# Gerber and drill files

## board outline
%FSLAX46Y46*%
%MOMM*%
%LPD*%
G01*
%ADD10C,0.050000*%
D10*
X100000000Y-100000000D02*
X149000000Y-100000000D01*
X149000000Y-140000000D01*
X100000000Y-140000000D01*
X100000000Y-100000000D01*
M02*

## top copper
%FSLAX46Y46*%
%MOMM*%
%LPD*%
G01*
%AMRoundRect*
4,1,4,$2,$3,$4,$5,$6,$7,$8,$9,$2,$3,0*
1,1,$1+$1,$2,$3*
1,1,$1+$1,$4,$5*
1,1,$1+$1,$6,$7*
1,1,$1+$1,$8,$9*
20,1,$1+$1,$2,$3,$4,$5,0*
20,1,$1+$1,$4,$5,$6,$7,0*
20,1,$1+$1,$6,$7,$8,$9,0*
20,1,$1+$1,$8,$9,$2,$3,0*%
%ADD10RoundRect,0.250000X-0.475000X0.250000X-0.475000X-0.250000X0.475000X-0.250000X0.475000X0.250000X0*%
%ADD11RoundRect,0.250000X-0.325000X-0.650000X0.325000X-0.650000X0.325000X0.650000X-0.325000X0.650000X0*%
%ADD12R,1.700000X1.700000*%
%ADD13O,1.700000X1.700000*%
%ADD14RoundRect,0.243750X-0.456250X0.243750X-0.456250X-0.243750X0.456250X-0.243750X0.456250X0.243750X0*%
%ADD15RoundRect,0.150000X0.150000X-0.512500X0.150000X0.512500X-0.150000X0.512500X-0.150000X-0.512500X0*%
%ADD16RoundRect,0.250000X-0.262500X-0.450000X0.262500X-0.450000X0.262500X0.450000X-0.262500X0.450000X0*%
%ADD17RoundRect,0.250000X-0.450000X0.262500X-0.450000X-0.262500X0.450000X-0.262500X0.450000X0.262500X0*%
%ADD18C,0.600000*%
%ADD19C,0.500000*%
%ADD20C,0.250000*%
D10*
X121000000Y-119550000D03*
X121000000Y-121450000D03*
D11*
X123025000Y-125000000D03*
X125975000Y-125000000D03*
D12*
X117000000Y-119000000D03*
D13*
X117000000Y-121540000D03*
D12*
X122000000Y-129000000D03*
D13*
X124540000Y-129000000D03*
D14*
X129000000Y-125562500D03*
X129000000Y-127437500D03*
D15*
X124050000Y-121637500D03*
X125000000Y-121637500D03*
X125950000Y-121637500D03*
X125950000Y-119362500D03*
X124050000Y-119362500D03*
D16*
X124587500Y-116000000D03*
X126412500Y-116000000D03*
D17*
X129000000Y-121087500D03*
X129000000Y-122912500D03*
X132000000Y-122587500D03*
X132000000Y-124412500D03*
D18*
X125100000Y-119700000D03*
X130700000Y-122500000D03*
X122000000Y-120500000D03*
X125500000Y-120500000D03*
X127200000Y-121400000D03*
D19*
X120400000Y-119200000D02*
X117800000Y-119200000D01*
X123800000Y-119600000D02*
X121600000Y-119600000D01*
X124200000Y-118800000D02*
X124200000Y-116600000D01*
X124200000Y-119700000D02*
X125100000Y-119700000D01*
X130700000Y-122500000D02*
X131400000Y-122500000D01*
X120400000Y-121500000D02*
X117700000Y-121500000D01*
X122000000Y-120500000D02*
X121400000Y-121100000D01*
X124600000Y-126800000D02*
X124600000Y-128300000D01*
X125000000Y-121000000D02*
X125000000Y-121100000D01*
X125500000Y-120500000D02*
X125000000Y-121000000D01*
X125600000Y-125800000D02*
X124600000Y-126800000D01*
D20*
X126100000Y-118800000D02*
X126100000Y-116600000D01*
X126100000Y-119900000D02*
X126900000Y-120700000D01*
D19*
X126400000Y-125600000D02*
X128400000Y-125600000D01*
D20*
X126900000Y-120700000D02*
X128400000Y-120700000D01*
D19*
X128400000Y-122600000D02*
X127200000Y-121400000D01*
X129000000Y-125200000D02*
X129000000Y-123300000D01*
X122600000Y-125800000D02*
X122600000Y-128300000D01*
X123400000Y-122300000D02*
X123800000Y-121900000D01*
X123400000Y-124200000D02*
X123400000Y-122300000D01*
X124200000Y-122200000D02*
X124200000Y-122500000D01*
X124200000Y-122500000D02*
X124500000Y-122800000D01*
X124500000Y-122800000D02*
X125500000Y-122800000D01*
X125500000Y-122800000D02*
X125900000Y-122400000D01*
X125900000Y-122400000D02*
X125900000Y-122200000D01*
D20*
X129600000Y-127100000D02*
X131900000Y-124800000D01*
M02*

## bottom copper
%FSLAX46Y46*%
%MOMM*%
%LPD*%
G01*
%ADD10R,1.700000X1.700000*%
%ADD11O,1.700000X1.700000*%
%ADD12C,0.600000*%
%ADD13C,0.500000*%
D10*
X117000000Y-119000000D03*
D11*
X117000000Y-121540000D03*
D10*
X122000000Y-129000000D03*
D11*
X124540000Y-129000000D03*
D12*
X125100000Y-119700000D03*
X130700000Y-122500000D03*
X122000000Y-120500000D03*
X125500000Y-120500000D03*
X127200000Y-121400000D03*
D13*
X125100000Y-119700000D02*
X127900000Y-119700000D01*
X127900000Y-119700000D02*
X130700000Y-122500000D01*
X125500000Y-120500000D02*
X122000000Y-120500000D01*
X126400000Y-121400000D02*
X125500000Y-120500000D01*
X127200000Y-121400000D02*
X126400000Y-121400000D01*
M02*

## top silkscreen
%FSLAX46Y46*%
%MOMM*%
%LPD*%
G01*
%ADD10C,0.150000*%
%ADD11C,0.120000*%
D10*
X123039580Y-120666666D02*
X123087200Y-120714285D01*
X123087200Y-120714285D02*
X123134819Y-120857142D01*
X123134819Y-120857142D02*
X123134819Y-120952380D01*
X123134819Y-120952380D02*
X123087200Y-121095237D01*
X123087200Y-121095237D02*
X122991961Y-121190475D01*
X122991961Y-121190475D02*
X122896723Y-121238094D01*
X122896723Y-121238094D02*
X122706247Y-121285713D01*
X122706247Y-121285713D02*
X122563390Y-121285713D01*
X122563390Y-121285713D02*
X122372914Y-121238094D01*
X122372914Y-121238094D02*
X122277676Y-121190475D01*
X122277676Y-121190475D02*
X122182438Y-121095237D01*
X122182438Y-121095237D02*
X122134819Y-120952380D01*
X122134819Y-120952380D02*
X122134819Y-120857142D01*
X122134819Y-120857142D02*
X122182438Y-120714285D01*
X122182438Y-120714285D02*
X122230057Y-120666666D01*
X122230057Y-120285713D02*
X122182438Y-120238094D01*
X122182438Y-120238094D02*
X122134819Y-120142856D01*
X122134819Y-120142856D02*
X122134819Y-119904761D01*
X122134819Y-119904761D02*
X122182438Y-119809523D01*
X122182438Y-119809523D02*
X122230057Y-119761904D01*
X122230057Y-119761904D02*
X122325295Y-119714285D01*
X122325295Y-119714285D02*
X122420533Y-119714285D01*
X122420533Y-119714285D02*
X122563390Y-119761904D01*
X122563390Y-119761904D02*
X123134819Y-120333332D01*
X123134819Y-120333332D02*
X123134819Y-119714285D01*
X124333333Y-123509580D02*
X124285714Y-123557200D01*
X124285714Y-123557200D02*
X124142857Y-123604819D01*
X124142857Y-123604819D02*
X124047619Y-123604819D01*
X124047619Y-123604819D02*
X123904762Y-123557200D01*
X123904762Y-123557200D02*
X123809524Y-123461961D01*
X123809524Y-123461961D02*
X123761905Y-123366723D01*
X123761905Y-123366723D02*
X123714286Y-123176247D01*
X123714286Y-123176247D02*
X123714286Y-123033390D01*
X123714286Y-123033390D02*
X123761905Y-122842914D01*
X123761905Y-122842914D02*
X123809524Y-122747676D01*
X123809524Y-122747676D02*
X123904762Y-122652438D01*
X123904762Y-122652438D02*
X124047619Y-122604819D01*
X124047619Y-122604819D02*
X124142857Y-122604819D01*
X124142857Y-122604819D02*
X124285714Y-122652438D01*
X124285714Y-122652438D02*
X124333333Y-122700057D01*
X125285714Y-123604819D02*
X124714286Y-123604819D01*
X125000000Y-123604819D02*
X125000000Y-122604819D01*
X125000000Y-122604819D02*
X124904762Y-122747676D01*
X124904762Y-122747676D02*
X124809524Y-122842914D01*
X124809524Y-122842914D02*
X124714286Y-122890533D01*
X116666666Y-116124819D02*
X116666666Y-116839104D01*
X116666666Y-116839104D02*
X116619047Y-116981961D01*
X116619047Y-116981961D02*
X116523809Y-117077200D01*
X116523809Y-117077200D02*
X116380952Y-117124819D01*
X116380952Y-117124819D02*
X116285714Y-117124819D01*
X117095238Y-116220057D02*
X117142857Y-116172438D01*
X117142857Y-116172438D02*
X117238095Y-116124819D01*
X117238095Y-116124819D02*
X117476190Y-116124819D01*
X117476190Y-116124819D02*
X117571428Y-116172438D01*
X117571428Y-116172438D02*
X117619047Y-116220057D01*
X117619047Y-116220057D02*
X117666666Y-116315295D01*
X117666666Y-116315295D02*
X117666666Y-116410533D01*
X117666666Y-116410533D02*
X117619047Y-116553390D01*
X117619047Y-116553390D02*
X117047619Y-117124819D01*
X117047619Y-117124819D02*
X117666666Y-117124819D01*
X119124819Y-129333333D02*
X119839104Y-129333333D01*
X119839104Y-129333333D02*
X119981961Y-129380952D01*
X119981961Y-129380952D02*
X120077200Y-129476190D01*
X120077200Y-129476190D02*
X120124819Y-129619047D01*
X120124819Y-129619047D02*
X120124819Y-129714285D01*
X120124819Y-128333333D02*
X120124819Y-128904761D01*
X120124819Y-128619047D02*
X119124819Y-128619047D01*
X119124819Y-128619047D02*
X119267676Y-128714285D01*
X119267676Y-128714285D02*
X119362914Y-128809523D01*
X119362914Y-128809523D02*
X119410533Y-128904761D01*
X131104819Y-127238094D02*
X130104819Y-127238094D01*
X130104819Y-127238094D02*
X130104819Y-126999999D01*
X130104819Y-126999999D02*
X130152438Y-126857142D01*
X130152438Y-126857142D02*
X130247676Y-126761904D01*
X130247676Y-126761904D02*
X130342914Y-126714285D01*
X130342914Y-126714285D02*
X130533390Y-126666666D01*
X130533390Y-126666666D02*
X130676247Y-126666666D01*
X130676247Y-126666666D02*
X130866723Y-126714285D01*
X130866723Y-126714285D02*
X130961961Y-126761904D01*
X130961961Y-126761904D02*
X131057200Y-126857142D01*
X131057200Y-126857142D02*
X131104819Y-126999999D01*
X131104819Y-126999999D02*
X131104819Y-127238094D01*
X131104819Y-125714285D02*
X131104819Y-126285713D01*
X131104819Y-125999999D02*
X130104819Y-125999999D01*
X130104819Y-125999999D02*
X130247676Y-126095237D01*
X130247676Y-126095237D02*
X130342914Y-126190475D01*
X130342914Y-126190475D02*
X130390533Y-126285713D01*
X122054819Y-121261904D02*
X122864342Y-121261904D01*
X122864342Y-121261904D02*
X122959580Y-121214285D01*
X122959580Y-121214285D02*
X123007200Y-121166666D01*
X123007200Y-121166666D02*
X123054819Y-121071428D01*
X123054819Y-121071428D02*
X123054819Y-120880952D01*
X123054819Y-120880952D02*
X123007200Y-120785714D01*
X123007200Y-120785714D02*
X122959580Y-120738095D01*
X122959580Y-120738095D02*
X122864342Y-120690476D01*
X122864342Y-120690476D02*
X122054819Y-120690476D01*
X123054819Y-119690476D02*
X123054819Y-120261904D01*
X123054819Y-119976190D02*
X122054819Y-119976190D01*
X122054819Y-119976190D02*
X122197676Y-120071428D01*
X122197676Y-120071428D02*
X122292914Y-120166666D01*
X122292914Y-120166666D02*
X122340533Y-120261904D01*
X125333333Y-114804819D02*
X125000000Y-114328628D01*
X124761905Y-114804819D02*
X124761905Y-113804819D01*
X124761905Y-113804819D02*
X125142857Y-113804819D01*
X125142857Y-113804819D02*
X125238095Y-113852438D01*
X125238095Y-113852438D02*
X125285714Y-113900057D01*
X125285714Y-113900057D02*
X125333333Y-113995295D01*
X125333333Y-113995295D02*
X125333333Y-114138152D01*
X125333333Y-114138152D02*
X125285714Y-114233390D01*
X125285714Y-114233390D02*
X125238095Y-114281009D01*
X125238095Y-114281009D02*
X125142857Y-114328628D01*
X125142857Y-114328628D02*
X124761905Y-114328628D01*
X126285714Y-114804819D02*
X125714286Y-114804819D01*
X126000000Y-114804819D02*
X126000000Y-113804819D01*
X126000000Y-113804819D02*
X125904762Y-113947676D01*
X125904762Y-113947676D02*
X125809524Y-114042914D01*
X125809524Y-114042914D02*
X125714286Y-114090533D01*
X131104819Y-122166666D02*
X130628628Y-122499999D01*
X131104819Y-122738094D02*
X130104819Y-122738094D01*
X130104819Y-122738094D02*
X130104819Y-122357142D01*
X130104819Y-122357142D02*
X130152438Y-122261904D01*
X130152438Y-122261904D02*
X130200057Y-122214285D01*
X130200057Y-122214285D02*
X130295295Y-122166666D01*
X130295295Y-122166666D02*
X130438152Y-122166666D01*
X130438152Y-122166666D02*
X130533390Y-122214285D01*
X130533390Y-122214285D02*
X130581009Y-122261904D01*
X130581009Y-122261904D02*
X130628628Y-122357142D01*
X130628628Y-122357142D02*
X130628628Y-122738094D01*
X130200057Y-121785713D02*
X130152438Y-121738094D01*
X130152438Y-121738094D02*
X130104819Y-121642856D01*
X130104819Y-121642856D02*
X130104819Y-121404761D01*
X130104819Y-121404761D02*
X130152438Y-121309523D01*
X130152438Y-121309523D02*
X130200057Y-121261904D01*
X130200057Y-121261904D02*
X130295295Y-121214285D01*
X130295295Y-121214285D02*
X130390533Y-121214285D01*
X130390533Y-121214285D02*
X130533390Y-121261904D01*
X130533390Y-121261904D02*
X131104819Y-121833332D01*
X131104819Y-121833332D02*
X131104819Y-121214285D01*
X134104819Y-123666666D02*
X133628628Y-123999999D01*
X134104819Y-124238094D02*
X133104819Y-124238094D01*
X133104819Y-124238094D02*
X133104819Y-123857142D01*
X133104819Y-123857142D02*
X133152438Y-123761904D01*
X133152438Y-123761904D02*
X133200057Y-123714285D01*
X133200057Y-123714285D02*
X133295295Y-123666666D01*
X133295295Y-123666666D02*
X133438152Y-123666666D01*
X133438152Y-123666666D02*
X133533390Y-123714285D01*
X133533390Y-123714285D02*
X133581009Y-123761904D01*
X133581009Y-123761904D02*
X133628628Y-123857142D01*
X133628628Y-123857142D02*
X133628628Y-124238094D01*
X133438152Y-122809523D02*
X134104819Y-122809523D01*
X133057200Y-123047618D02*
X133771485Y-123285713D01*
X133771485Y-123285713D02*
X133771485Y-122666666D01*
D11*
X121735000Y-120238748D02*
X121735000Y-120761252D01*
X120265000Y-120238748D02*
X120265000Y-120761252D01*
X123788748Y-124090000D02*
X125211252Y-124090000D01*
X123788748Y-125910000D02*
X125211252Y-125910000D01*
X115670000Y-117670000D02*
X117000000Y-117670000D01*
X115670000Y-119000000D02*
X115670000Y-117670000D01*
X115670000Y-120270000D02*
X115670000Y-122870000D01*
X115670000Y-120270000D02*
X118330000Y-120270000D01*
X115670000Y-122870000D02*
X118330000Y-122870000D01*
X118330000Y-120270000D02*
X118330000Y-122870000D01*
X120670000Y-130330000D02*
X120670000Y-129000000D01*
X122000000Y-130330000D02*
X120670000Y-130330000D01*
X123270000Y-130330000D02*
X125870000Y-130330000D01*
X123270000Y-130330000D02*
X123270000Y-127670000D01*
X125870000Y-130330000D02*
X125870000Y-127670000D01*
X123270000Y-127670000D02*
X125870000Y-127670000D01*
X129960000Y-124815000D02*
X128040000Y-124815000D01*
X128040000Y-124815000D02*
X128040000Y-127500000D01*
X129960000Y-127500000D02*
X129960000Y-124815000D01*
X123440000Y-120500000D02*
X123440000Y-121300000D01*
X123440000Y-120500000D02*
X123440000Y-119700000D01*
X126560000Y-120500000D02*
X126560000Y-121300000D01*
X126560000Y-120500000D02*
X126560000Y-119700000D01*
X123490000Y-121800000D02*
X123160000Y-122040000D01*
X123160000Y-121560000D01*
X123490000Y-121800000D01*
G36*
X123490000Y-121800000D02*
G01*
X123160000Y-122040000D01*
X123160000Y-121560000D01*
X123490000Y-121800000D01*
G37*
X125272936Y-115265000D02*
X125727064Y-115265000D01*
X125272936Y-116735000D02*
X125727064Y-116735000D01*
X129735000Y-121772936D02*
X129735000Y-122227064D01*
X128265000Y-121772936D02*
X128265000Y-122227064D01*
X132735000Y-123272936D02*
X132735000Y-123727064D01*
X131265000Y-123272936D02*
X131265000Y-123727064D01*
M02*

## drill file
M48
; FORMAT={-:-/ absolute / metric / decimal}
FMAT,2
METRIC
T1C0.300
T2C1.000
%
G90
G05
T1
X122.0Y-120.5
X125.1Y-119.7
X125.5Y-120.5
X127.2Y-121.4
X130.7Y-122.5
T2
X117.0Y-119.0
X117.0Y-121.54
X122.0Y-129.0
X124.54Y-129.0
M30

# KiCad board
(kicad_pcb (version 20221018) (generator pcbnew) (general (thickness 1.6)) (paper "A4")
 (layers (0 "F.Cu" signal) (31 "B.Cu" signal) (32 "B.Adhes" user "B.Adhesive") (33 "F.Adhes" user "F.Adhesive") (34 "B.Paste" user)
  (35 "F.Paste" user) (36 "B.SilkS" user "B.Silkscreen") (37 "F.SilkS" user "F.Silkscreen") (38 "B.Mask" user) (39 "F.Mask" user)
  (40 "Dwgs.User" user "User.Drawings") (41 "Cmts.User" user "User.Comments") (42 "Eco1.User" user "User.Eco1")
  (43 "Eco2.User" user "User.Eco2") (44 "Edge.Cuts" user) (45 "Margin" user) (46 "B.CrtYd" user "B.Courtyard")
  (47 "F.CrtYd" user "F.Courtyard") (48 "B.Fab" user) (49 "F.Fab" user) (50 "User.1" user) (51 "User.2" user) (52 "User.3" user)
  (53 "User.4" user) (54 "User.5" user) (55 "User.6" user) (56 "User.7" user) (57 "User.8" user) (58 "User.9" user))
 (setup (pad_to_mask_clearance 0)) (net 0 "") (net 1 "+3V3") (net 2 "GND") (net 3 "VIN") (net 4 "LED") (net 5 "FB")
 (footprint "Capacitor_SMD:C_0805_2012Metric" (layer "F.Cu") (at 121 120.5 -90)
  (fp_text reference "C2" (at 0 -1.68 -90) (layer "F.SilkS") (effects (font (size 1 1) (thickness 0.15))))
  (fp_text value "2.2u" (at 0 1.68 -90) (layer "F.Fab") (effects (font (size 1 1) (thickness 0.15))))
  (fp_line (start -0.261252 -0.735) (end 0.261252 -0.735) (stroke (width 0.12) (type solid)) (layer "F.SilkS"))
  (fp_line (start -0.261252 0.735) (end 0.261252 0.735) (stroke (width 0.12) (type solid)) (layer "F.SilkS"))
  (pad "1" smd roundrect (at -0.95 0 270) (size 1 1.45) (layers "F.Cu" "F.Paste" "F.Mask") (roundrect_rratio 0.25) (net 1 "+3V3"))
  (pad "2" smd roundrect (at 0.95 0 270) (size 1 1.45) (layers "F.Cu" "F.Paste" "F.Mask") (roundrect_rratio 0.25) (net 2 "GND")))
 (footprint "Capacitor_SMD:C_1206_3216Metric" (layer "F.Cu") (at 124.5 125)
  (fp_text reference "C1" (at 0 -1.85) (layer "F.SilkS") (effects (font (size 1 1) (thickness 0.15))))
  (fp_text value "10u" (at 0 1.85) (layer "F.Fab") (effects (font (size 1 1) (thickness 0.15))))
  (fp_line (start -0.711252 -0.91) (end 0.711252 -0.91) (stroke (width 0.12) (type solid)) (layer "F.SilkS"))
  (fp_line (start -0.711252 0.91) (end 0.711252 0.91) (stroke (width 0.12) (type solid)) (layer "F.SilkS"))
  (pad "1" smd roundrect (at -1.475 0) (size 1.15 1.8) (layers "F.Cu" "F.Paste" "F.Mask") (roundrect_rratio 0.217391) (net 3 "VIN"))
  (pad "2" smd roundrect (at 1.475 0) (size 1.15 1.8) (layers "F.Cu" "F.Paste" "F.Mask") (roundrect_rratio 0.217391) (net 2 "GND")))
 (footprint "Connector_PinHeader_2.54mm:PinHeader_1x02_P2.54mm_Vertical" (layer "F.Cu") (at 117 119)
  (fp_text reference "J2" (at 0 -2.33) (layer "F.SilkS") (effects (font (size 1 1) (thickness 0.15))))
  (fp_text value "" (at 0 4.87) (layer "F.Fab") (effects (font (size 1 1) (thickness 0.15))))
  (fp_line (start -1.33 -1.33) (end 0 -1.33) (stroke (width 0.12) (type solid)) (layer "F.SilkS"))
  (fp_line (start -1.33 0) (end -1.33 -1.33) (stroke (width 0.12) (type solid)) (layer "F.SilkS"))
  (fp_line (start -1.33 1.27) (end -1.33 3.87) (stroke (width 0.12) (type solid)) (layer "F.SilkS"))
  (fp_line (start -1.33 1.27) (end 1.33 1.27) (stroke (width 0.12) (type solid)) (layer "F.SilkS"))
  (fp_line (start -1.33 3.87) (end 1.33 3.87) (stroke (width 0.12) (type solid)) (layer "F.SilkS"))
  (fp_line (start 1.33 1.27) (end 1.33 3.87) (stroke (width 0.12) (type solid)) (layer "F.SilkS"))
  (pad "1" thru_hole rect (at 0 0) (size 1.7 1.7) (drill 1) (layers "*.Cu" "*.Mask") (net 1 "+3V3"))
  (pad "2" thru_hole oval (at 0 2.54) (size 1.7 1.7) (drill 1) (layers "*.Cu" "*.Mask") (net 2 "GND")))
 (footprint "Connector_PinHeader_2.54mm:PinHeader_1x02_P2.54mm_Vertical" (layer "F.Cu") (at 122 129 90)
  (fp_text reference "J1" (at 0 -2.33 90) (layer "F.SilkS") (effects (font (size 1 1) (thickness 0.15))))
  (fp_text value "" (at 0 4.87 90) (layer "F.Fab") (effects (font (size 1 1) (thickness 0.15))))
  (fp_line (start -1.33 -1.33) (end 0 -1.33) (stroke (width 0.12) (type solid)) (layer "F.SilkS"))
  (fp_line (start -1.33 0) (end -1.33 -1.33) (stroke (width 0.12) (type solid)) (layer "F.SilkS"))
  (fp_line (start -1.33 1.27) (end -1.33 3.87) (stroke (width 0.12) (type solid)) (layer "F.SilkS"))
  (fp_line (start -1.33 1.27) (end 1.33 1.27) (stroke (width 0.12) (type solid)) (layer "F.SilkS"))
  (fp_line (start -1.33 3.87) (end 1.33 3.87) (stroke (width 0.12) (type solid)) (layer "F.SilkS"))
  (fp_line (start 1.33 1.27) (end 1.33 3.87) (stroke (width 0.12) (type solid)) (layer "F.SilkS"))
  (pad "1" thru_hole rect (at 0 0 90) (size 1.7 1.7) (drill 1) (layers "*.Cu" "*.Mask") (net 3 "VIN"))
  (pad "2" thru_hole oval (at 0 2.54 90) (size 1.7 1.7) (drill 1) (layers "*.Cu" "*.Mask") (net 2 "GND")))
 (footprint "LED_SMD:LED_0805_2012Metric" (layer "F.Cu") (at 129 126.5 -90)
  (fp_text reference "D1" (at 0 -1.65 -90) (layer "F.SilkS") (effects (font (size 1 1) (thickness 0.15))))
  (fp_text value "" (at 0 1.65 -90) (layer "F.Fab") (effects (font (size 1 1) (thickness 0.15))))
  (fp_line (start -1.685 -0.96) (end -1.685 0.96) (stroke (width 0.12) (type solid)) (layer "F.SilkS"))
  (fp_line (start -1.685 0.96) (end 1 0.96) (stroke (width 0.12) (type solid)) (layer "F.SilkS"))
  (fp_line (start 1 -0.96) (end -1.685 -0.96) (stroke (width 0.12) (type solid)) (layer "F.SilkS"))
  (pad "1" smd roundrect (at -0.9375 0 270) (size 0.975 1.4) (layers "F.Cu" "F.Paste" "F.Mask") (roundrect_rratio 0.25) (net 2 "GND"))
  (pad "2" smd roundrect (at 0.9375 0 270) (size 0.975 1.4) (layers "F.Cu" "F.Paste" "F.Mask") (roundrect_rratio 0.25) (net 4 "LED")))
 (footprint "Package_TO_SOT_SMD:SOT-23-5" (layer "F.Cu") (at 125 120.5 90)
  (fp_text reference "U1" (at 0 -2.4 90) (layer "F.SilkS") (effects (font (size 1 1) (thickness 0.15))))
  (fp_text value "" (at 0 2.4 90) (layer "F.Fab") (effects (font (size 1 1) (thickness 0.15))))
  (fp_line (start 0 -1.56) (end -0.8 -1.56) (stroke (width 0.12) (type solid)) (layer "F.SilkS"))
  (fp_line (start 0 -1.56) (end 0.8 -1.56) (stroke (width 0.12) (type solid)) (layer "F.SilkS"))
  (fp_line (start 0 1.56) (end -0.8 1.56) (stroke (width 0.12) (type solid)) (layer "F.SilkS"))
  (fp_line (start 0 1.56) (end 0.8 1.56) (stroke (width 0.12) (type solid)) (layer "F.SilkS"))
  (fp_poly
   (pts (xy -1.3 -1.51) (xy -1.54 -1.84) (xy -1.06 -1.84) (xy -1.3 -1.51)) (stroke (width 0.12) (type solid)) (fill solid) (layer "F.SilkS"))
  (pad "1" smd roundrect (at -1.1375 -0.95 90) (size 1.325 0.6) (layers "F.Cu" "F.Paste" "F.Mask") (roundrect_rratio 0.25) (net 3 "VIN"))
  (pad "2" smd roundrect (at -1.1375 0 90) (size 1.325 0.6) (layers "F.Cu" "F.Paste" "F.Mask") (roundrect_rratio 0.25) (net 2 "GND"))
  (pad "3" smd roundrect (at -1.1375 0.95 90) (size 1.325 0.6) (layers "F.Cu" "F.Paste" "F.Mask") (roundrect_rratio 0.25) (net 3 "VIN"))
  (pad "4" smd roundrect (at 1.1375 0.95 90) (size 1.325 0.6) (layers "F.Cu" "F.Paste" "F.Mask") (roundrect_rratio 0.25) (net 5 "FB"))
  (pad "5" smd roundrect (at 1.1375 -0.95 90) (size 1.325 0.6) (layers "F.Cu" "F.Paste" "F.Mask") (roundrect_rratio 0.25) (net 1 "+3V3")))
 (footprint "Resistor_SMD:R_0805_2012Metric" (layer "F.Cu") (at 125.5 116)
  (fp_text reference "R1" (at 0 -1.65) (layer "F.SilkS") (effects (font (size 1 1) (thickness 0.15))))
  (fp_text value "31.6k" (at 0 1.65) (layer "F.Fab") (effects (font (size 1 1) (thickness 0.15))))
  (fp_line (start -0.227064 -0.735) (end 0.227064 -0.735) (stroke (width 0.12) (type solid)) (layer "F.SilkS"))
  (fp_line (start -0.227064 0.735) (end 0.227064 0.735) (stroke (width 0.12) (type solid)) (layer "F.SilkS"))
  (pad "1" smd roundrect (at -0.9125 0) (size 1.025 1.4) (layers "F.Cu" "F.Paste" "F.Mask") (roundrect_rratio 0.243902) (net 1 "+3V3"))
  (pad "2" smd roundrect (at 0.9125 0) (size 1.025 1.4) (layers "F.Cu" "F.Paste" "F.Mask") (roundrect_rratio 0.243902) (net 5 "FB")))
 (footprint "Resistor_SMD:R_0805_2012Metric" (layer "F.Cu") (at 129 122 -90)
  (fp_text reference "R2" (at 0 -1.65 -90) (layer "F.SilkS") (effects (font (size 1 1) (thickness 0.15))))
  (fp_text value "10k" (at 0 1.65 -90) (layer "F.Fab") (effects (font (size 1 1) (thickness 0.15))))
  (fp_line (start -0.227064 -0.735) (end 0.227064 -0.735) (stroke (width 0.12) (type solid)) (layer "F.SilkS"))
  (fp_line (start -0.227064 0.735) (end 0.227064 0.735) (stroke (width 0.12) (type solid)) (layer "F.SilkS"))
  (pad "1" smd roundrect (at -0.9125 0 270) (size 1.025 1.4) (layers "F.Cu" "F.Paste" "F.Mask") (roundrect_rratio 0.243902) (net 5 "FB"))
  (pad "2" smd roundrect (at 0.9125 0 270) (size 1.025 1.4) (layers "F.Cu" "F.Paste" "F.Mask") (roundrect_rratio 0.243902) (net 2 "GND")))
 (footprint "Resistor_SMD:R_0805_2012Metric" (layer "F.Cu") (at 132 123.5 -90)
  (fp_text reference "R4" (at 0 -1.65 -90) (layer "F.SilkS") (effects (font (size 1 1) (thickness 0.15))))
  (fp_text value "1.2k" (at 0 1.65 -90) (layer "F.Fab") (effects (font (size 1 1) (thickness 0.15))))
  (fp_line (start -0.227064 -0.735) (end 0.227064 -0.735) (stroke (width 0.12) (type solid)) (layer "F.SilkS"))
  (fp_line (start -0.227064 0.735) (end 0.227064 0.735) (stroke (width 0.12) (type solid)) (layer "F.SilkS"))
  (pad "1" smd roundrect (at -0.9125 0 270) (size 1.025 1.4) (layers "F.Cu" "F.Paste" "F.Mask") (roundrect_rratio 0.243902) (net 1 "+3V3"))
  (pad "2" smd roundrect (at 0.9125 0 270) (size 1.025 1.4) (layers "F.Cu" "F.Paste" "F.Mask") (roundrect_rratio 0.243902) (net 4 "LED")))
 (gr_rect (start 100 100) (end 149 140) (stroke (width 0.05) (type default)) (fill none) (layer "Edge.Cuts"))
 (segment (start 120.4 119.2) (end 117.8 119.2) (width 0.5) (layer "F.Cu") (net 1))
 (segment (start 123.8 119.6) (end 121.6 119.6) (width 0.5) (layer "F.Cu") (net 1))
 (segment (start 124.2 118.8) (end 124.2 116.6) (width 0.5) (layer "F.Cu") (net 1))
 (segment (start 124.2 119.7) (end 125.1 119.7) (width 0.5) (layer "F.Cu") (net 1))
 (segment (start 130.7 122.5) (end 131.4 122.5) (width 0.5) (layer "F.Cu") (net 1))
 (via (at 125.1 119.7) (size 0.6) (drill 0.3) (layers "F.Cu" "B.Cu") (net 1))
 (via (at 130.7 122.5) (size 0.6) (drill 0.3) (layers "F.Cu" "B.Cu") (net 1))
 (segment (start 120.4 121.5) (end 117.7 121.5) (width 0.5) (layer "F.Cu") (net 2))
 (segment (start 122 120.5) (end 121.4 121.1) (width 0.5) (layer "F.Cu") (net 2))
 (segment (start 124.6 126.8) (end 124.6 128.3) (width 0.5) (layer "F.Cu") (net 2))
 (segment (start 125 121) (end 125 121.1) (width 0.5) (layer "F.Cu") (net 2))
 (segment (start 125.1 119.7) (end 127.9 119.7) (width 0.5) (layer "B.Cu") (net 1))
 (segment (start 125.5 120.5) (end 125 121) (width 0.5) (layer "F.Cu") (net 2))
 (segment (start 125.6 125.8) (end 124.6 126.8) (width 0.5) (layer "F.Cu") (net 2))
 (segment (start 126.1 118.8) (end 126.1 116.6) (width 0.25) (layer "F.Cu") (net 5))
 (segment (start 126.1 119.9) (end 126.9 120.7) (width 0.25) (layer "F.Cu") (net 5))
 (segment (start 126.4 125.6) (end 128.4 125.6) (width 0.5) (layer "F.Cu") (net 2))
 (segment (start 126.9 120.7) (end 128.4 120.7) (width 0.25) (layer "F.Cu") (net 5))
 (segment (start 127.9 119.7) (end 130.7 122.5) (width 0.5) (layer "B.Cu") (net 1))
 (segment (start 128.4 122.6) (end 127.2 121.4) (width 0.5) (layer "F.Cu") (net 2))
 (segment (start 129 125.2) (end 129 123.3) (width 0.5) (layer "F.Cu") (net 2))
 (via (at 122 120.5) (size 0.6) (drill 0.3) (layers "F.Cu" "B.Cu") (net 2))
 (via (at 125.5 120.5) (size 0.6) (drill 0.3) (layers "F.Cu" "B.Cu") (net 2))
 (via (at 127.2 121.4) (size 0.6) (drill 0.3) (layers "F.Cu" "B.Cu") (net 2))
 (segment (start 122.6 125.8) (end 122.6 128.3) (width 0.5) (layer "F.Cu") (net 3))
 (segment (start 123.4 122.3) (end 123.8 121.9) (width 0.5) (layer "F.Cu") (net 3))
 (segment (start 123.4 124.2) (end 123.4 122.3) (width 0.5) (layer "F.Cu") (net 3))
 (segment (start 124.2 122.2) (end 124.2 122.5) (width 0.5) (layer "F.Cu") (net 3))
 (segment (start 124.2 122.5) (end 124.5 122.8) (width 0.5) (layer "F.Cu") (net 3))
 (segment (start 124.5 122.8) (end 125.5 122.8) (width 0.5) (layer "F.Cu") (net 3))
 (segment (start 125.5 120.5) (end 122 120.5) (width 0.5) (layer "B.Cu") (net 2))
 (segment (start 125.5 122.8) (end 125.9 122.4) (width 0.5) (layer "F.Cu") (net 3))
 (segment (start 125.9 122.4) (end 125.9 122.2) (width 0.5) (layer "F.Cu") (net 3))
 (segment (start 126.4 121.4) (end 125.5 120.5) (width 0.5) (layer "B.Cu") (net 2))
 (segment (start 127.2 121.4) (end 126.4 121.4) (width 0.5) (layer "B.Cu") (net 2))
 (segment (start 129.6 127.1) (end 131.9 124.8) (width 0.25) (layer "F.Cu") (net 4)))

